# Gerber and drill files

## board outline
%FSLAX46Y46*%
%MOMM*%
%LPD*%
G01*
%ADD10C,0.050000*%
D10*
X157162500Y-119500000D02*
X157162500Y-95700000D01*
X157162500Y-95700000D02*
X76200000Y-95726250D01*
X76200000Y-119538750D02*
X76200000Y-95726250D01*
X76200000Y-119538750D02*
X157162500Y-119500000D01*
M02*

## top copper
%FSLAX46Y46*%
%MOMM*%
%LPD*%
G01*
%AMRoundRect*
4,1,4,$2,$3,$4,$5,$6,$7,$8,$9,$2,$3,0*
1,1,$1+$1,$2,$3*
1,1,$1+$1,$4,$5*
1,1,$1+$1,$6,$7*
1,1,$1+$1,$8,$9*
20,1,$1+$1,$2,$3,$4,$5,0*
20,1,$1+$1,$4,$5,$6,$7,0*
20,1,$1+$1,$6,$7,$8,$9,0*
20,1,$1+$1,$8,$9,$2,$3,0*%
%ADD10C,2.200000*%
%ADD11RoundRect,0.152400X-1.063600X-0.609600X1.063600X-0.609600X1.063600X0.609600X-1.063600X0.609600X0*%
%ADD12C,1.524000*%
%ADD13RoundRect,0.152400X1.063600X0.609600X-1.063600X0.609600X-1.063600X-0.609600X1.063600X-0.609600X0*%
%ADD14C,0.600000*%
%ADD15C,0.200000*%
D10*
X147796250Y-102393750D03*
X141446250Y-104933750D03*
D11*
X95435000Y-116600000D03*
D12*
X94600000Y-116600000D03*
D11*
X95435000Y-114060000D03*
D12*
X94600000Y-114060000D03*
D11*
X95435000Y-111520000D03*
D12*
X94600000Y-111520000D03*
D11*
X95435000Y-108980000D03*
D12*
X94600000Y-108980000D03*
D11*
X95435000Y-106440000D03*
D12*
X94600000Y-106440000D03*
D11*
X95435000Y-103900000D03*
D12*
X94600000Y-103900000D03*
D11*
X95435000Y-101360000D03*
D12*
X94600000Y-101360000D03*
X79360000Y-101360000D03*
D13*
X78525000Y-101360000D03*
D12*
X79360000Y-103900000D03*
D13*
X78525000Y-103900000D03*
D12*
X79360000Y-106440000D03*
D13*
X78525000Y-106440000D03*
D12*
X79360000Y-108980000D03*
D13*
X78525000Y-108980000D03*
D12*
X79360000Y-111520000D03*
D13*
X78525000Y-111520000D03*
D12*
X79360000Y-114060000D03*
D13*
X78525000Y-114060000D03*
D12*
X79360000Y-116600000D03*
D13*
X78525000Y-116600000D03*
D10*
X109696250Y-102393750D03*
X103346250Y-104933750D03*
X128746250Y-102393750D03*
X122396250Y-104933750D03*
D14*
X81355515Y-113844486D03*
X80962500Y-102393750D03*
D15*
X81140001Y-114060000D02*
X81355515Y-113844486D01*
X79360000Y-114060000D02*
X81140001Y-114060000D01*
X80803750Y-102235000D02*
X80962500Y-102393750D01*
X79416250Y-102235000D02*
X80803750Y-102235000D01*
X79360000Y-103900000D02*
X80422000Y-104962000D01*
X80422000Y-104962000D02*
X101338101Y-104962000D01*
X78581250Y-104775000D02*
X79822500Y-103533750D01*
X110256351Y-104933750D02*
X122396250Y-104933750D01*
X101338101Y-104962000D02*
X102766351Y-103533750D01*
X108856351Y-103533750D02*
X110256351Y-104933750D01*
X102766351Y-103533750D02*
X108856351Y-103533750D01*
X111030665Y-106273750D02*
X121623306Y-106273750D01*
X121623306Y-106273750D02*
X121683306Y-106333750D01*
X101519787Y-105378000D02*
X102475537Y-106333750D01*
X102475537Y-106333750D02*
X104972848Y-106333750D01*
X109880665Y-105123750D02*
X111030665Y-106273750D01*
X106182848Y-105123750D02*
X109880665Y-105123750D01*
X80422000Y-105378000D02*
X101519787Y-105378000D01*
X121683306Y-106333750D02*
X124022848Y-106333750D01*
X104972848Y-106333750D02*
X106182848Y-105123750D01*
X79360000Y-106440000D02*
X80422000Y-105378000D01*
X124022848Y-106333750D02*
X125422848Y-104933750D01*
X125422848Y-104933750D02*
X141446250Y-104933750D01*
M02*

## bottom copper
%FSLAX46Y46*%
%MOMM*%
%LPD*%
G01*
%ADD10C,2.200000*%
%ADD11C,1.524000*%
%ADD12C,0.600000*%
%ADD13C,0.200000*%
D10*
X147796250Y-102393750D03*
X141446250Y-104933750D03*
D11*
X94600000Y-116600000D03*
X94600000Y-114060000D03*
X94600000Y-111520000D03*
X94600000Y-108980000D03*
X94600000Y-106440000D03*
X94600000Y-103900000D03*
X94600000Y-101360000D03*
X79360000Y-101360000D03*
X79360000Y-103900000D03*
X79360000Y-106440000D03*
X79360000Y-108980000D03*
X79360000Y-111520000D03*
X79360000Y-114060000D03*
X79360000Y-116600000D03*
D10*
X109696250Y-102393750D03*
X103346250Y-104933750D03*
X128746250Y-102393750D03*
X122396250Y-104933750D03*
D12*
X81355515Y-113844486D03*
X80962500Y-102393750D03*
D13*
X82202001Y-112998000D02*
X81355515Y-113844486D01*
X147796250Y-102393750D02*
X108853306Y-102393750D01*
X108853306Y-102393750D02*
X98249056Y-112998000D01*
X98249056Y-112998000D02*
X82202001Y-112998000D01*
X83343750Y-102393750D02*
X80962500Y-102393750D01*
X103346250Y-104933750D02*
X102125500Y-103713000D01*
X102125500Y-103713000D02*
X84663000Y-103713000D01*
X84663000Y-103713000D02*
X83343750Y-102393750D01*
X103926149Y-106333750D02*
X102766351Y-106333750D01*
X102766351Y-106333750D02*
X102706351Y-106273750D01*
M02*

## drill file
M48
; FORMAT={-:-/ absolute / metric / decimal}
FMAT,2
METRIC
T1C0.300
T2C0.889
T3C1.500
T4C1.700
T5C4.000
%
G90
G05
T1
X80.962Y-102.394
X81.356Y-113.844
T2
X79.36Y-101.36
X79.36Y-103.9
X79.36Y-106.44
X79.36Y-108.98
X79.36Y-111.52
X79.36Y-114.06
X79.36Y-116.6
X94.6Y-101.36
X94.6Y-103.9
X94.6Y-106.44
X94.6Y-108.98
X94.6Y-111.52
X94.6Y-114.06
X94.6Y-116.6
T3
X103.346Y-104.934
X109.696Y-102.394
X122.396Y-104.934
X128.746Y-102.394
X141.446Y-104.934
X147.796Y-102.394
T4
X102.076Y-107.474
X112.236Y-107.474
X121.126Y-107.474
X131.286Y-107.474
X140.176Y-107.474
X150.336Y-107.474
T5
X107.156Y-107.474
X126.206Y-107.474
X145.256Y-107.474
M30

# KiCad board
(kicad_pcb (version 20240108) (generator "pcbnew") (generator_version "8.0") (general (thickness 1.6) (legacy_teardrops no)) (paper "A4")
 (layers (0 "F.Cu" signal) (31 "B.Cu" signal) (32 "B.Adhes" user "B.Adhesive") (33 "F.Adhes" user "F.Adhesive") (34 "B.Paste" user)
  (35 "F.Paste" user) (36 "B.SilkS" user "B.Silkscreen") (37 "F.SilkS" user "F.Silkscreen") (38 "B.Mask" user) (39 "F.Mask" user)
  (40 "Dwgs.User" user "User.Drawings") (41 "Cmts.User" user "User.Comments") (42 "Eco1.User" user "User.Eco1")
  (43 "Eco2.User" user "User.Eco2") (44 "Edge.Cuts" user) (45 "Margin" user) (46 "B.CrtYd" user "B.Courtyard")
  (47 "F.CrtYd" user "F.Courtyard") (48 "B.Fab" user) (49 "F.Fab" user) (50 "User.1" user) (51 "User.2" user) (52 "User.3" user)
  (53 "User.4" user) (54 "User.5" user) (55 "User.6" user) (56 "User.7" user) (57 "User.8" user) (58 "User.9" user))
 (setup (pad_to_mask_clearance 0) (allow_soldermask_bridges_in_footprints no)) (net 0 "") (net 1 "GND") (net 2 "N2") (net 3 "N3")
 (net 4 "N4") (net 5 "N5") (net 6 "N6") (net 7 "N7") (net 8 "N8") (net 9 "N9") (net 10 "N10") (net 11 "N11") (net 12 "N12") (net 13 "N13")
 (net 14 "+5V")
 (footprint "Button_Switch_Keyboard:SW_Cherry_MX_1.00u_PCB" (layer "F.Cu") (at 147.79625 102.39375)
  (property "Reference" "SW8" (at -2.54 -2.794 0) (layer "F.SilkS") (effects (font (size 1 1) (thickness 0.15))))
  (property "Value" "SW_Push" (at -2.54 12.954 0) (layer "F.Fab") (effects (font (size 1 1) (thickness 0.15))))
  (pad "" np_thru_hole circle (at -7.62 5.08) (size 1.7 1.7) (drill 1.7) (layers "*.Cu" "*.Mask"))
  (pad "" np_thru_hole circle (at -2.54 5.08) (size 4 4) (drill 4) (layers "*.Cu" "*.Mask"))
  (pad "" np_thru_hole circle (at 2.54 5.08) (size 1.7 1.7) (drill 1.7) (layers "*.Cu" "*.Mask"))
  (pad "1" thru_hole circle (at 0 0) (size 2.2 2.2) (drill 1.5) (layers "*.Cu" "*.Mask") (remove_unused_layers no) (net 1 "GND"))
  (pad "2" thru_hole circle (at -6.35 2.54) (size 2.2 2.2) (drill 1.5) (layers "*.Cu" "*.Mask") (remove_unused_layers no) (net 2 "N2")))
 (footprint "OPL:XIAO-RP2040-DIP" (layer "F.Cu") (at 86.98 108.98 180)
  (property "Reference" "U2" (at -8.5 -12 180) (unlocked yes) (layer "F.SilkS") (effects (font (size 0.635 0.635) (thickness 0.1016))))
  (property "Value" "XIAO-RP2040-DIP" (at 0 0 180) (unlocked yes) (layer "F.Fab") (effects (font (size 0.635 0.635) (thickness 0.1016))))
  (pad "1" smd roundrect (at -8.455 -7.62) (size 2.432 1.524) (layers "F.Cu" "F.Mask") (roundrect_rratio 0.1) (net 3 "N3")
   (thermal_bridge_angle 45))
  (pad "1" thru_hole circle (at -7.62 -7.62) (size 1.524 1.524) (drill 0.889) (layers "*.Cu" "*.Mask") (remove_unused_layers no)
   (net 3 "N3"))
  (pad "2" smd roundrect (at -8.455 -5.08) (size 2.432 1.524) (layers "F.Cu" "F.Mask") (roundrect_rratio 0.1) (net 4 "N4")
   (thermal_bridge_angle 45))
  (pad "2" thru_hole circle (at -7.62 -5.08) (size 1.524 1.524) (drill 0.889) (layers "*.Cu" "*.Mask") (remove_unused_layers no)
   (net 4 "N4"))
  (pad "3" smd roundrect (at -8.455 -2.54) (size 2.432 1.524) (layers "F.Cu" "F.Mask") (roundrect_rratio 0.1) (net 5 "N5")
   (thermal_bridge_angle 45))
  (pad "3" thru_hole circle (at -7.62 -2.54) (size 1.524 1.524) (drill 0.889) (layers "*.Cu" "*.Mask") (remove_unused_layers no)
   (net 5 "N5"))
  (pad "4" smd roundrect (at -8.455 0) (size 2.432 1.524) (layers "F.Cu" "F.Mask") (roundrect_rratio 0.1) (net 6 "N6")
   (thermal_bridge_angle 45))
  (pad "4" thru_hole circle (at -7.62 0) (size 1.524 1.524) (drill 0.889) (layers "*.Cu" "*.Mask") (remove_unused_layers no) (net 6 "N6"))
  (pad "5" smd roundrect (at -8.455 2.54) (size 2.432 1.524) (layers "F.Cu" "F.Mask") (roundrect_rratio 0.1) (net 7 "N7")
   (thermal_bridge_angle 45))
  (pad "5" thru_hole circle (at -7.62 2.54) (size 1.524 1.524) (drill 0.889) (layers "*.Cu" "*.Mask") (remove_unused_layers no) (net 7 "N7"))
  (pad "6" smd roundrect (at -8.455 5.08) (size 2.432 1.524) (layers "F.Cu" "F.Mask") (roundrect_rratio 0.1) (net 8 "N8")
   (thermal_bridge_angle 45))
  (pad "6" thru_hole circle (at -7.62 5.08) (size 1.524 1.524) (drill 0.889) (layers "*.Cu" "*.Mask") (remove_unused_layers no) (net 8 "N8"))
  (pad "7" smd roundrect (at -8.455 7.62) (size 2.432 1.524) (layers "F.Cu" "F.Mask") (roundrect_rratio 0.1) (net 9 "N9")
   (thermal_bridge_angle 45))
  (pad "7" thru_hole circle (at -7.62 7.62) (size 1.524 1.524) (drill 0.889) (layers "*.Cu" "*.Mask") (remove_unused_layers no) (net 9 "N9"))
  (pad "8" thru_hole circle (at 7.62 7.62 180) (size 1.524 1.524) (drill 0.889) (layers "*.Cu" "*.Mask") (remove_unused_layers no)
   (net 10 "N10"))
  (pad "8" smd roundrect (at 8.455 7.62 180) (size 2.432 1.524) (layers "F.Cu" "F.Mask") (roundrect_rratio 0.1) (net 10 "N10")
   (thermal_bridge_angle 45))
  (pad "9" thru_hole circle (at 7.62 5.08 180) (size 1.524 1.524) (drill 0.889) (layers "*.Cu" "*.Mask") (remove_unused_layers no)
   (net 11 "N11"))
  (pad "9" smd roundrect (at 8.455 5.08 180) (size 2.432 1.524) (layers "F.Cu" "F.Mask") (roundrect_rratio 0.1) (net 11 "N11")
   (thermal_bridge_angle 45))
  (pad "10" thru_hole circle (at 7.62 2.54 180) (size 1.524 1.524) (drill 0.889) (layers "*.Cu" "*.Mask") (remove_unused_layers no)
   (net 2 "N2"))
  (pad "10" smd roundrect (at 8.455 2.54 180) (size 2.432 1.524) (layers "F.Cu" "F.Mask") (roundrect_rratio 0.1) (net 2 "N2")
   (thermal_bridge_angle 45))
  (pad "11" thru_hole circle (at 7.62 0 180) (size 1.524 1.524) (drill 0.889) (layers "*.Cu" "*.Mask") (remove_unused_layers no)
   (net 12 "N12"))
  (pad "11" smd roundrect (at 8.455 0 180) (size 2.432 1.524) (layers "F.Cu" "F.Mask") (roundrect_rratio 0.1) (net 12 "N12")
   (thermal_bridge_angle 45))
  (pad "12" thru_hole circle (at 7.62 -2.54 180) (size 1.524 1.524) (drill 0.889) (layers "*.Cu" "*.Mask") (remove_unused_layers no)
   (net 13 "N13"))
  (pad "12" smd roundrect (at 8.455 -2.54 180) (size 2.432 1.524) (layers "F.Cu" "F.Mask") (roundrect_rratio 0.1) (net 13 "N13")
   (thermal_bridge_angle 45))
  (pad "13" thru_hole circle (at 7.62 -5.08 180) (size 1.524 1.524) (drill 0.889) (layers "*.Cu" "*.Mask") (remove_unused_layers no)
   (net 1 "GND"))
  (pad "13" smd roundrect (at 8.455 -5.08 180) (size 2.432 1.524) (layers "F.Cu" "F.Mask") (roundrect_rratio 0.1) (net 1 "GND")
   (thermal_bridge_angle 45))
  (pad "14" thru_hole circle (at 7.62 -7.62 180) (size 1.524 1.524) (drill 0.889) (layers "*.Cu" "*.Mask") (remove_unused_layers no)
   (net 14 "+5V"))
  (pad "14" smd roundrect (at 8.455 -7.62 180) (size 2.432 1.524) (layers "F.Cu" "F.Mask") (roundrect_rratio 0.1) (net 14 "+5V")
   (thermal_bridge_angle 45)))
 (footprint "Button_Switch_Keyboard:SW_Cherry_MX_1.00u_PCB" (layer "F.Cu") (at 109.69625 102.39375)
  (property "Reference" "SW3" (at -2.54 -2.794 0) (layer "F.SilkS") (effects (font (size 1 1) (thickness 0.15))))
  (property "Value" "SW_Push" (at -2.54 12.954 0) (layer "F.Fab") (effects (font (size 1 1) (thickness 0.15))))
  (pad "" np_thru_hole circle (at -7.62 5.08) (size 1.7 1.7) (drill 1.7) (layers "*.Cu" "*.Mask"))
  (pad "" np_thru_hole circle (at -2.54 5.08) (size 4 4) (drill 4) (layers "*.Cu" "*.Mask"))
  (pad "" np_thru_hole circle (at 2.54 5.08) (size 1.7 1.7) (drill 1.7) (layers "*.Cu" "*.Mask"))
  (pad "1" thru_hole circle (at 0 0) (size 2.2 2.2) (drill 1.5) (layers "*.Cu" "*.Mask") (remove_unused_layers no) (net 1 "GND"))
  (pad "2" thru_hole circle (at -6.35 2.54) (size 2.2 2.2) (drill 1.5) (layers "*.Cu" "*.Mask") (remove_unused_layers no) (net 10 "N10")))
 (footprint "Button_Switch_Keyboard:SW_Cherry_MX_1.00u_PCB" (layer "F.Cu") (at 128.74625 102.39375)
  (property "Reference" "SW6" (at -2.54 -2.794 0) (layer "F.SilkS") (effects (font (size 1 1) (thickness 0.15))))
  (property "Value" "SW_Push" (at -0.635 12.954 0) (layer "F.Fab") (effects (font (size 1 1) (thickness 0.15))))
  (pad "" np_thru_hole circle (at -7.62 5.08) (size 1.7 1.7) (drill 1.7) (layers "*.Cu" "*.Mask"))
  (pad "" np_thru_hole circle (at -2.54 5.08) (size 4 4) (drill 4) (layers "*.Cu" "*.Mask"))
  (pad "" np_thru_hole circle (at 2.54 5.08) (size 1.7 1.7) (drill 1.7) (layers "*.Cu" "*.Mask"))
  (pad "1" thru_hole circle (at 0 0) (size 2.2 2.2) (drill 1.5) (layers "*.Cu" "*.Mask") (remove_unused_layers no) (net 1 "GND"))
  (pad "2" thru_hole circle (at -6.35 2.54) (size 2.2 2.2) (drill 1.5) (layers "*.Cu" "*.Mask") (remove_unused_layers no) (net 11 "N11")))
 (gr_line (start 157.1625 119.5) (end 157.1625 95.7) (stroke (width 0.05) (type default)) (layer "Edge.Cuts"))
 (gr_line (start 157.1625 95.7) (end 76.2 95.72625) (stroke (width 0.05) (type default)) (layer "Edge.Cuts"))
 (gr_line (start 76.2 119.53875) (end 76.2 95.72625) (stroke (width 0.05) (type default)) (layer "Edge.Cuts"))
 (gr_line (start 76.2 119.53875) (end 157.1625 119.5) (stroke (width 0.05) (type default)) (layer "Edge.Cuts"))
 (segment (start 81.140001 114.06) (end 81.355515 113.844486) (width 0.2) (layer "F.Cu") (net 1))
 (segment (start 79.36 114.06) (end 81.140001 114.06) (width 0.2) (layer "F.Cu") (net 1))
 (via (at 81.355515 113.844486) (size 0.6) (drill 0.3) (layers "F.Cu" "B.Cu") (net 1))
 (segment (start 82.202001 112.998) (end 81.355515 113.844486) (width 0.2) (layer "B.Cu") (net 1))
 (segment (start 147.79625 102.39375) (end 108.853306 102.39375) (width 0.2) (layer "B.Cu") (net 1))
 (segment (start 108.853306 102.39375) (end 98.249056 112.998) (width 0.2) (layer "B.Cu") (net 1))
 (segment (start 98.249056 112.998) (end 82.202001 112.998) (width 0.2) (layer "B.Cu") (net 1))
 (segment (start 80.80375 102.235) (end 80.9625 102.39375) (width 0.2) (layer "F.Cu") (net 10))
 (segment (start 79.41625 102.235) (end 80.80375 102.235) (width 0.2) (layer "F.Cu") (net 10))
 (via (at 80.9625 102.39375) (size 0.6) (drill 0.3) (layers "F.Cu" "B.Cu") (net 10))
 (segment (start 83.34375 102.39375) (end 80.9625 102.39375) (width 0.2) (layer "B.Cu") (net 10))
 (segment (start 103.34625 104.93375) (end 102.1255 103.713) (width 0.2) (layer "B.Cu") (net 10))
 (segment (start 102.1255 103.713) (end 84.663 103.713) (width 0.2) (layer "B.Cu") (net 10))
 (segment (start 84.663 103.713) (end 83.34375 102.39375) (width 0.2) (layer "B.Cu") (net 10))
 (segment (start 79.36 103.9) (end 80.422 104.962) (width 0.2) (layer "F.Cu") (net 11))
 (segment (start 80.422 104.962) (end 101.338101 104.962) (width 0.2) (layer "F.Cu") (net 11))
 (segment (start 78.58125 104.775) (end 79.8225 103.53375) (width 0.2) (layer "F.Cu") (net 11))
 (segment (start 110.256351 104.93375) (end 122.39625 104.93375) (width 0.2) (layer "F.Cu") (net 11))
 (segment (start 101.338101 104.962) (end 102.766351 103.53375) (width 0.2) (layer "F.Cu") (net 11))
 (segment (start 108.856351 103.53375) (end 110.256351 104.93375) (width 0.2) (layer "F.Cu") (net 11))
 (segment (start 102.766351 103.53375) (end 108.856351 103.53375) (width 0.2) (layer "F.Cu") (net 11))
 (segment (start 111.030665 106.27375) (end 121.623306 106.27375) (width 0.2) (layer "F.Cu") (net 2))
 (segment (start 121.623306 106.27375) (end 121.683306 106.33375) (width 0.2) (layer "F.Cu") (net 2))
 (segment (start 101.519787 105.378) (end 102.475537 106.33375) (width 0.2) (layer "F.Cu") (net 2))
 (segment (start 102.475537 106.33375) (end 104.972848 106.33375) (width 0.2) (layer "F.Cu") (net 2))
 (segment (start 109.880665 105.12375) (end 111.030665 106.27375) (width 0.2) (layer "F.Cu") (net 2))
 (segment (start 106.182848 105.12375) (end 109.880665 105.12375) (width 0.2) (layer "F.Cu") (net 2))
 (segment (start 80.422 105.378) (end 101.519787 105.378) (width 0.2) (layer "F.Cu") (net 2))
 (segment (start 121.683306 106.33375) (end 124.022848 106.33375) (width 0.2) (layer "F.Cu") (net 2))
 (segment (start 104.972848 106.33375) (end 106.182848 105.12375) (width 0.2) (layer "F.Cu") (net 2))
 (segment (start 79.36 106.44) (end 80.422 105.378) (width 0.2) (layer "F.Cu") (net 2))
 (segment (start 124.022848 106.33375) (end 125.422848 104.93375) (width 0.2) (layer "F.Cu") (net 2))
 (segment (start 125.422848 104.93375) (end 141.44625 104.93375) (width 0.2) (layer "F.Cu") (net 2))
 (segment (start 103.926149 106.33375) (end 102.766351 106.33375) (width 0.2) (layer "B.Cu") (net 5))
 (segment (start 102.766351 106.33375) (end 102.706351 106.27375) (width 0.2) (layer "B.Cu") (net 5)))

